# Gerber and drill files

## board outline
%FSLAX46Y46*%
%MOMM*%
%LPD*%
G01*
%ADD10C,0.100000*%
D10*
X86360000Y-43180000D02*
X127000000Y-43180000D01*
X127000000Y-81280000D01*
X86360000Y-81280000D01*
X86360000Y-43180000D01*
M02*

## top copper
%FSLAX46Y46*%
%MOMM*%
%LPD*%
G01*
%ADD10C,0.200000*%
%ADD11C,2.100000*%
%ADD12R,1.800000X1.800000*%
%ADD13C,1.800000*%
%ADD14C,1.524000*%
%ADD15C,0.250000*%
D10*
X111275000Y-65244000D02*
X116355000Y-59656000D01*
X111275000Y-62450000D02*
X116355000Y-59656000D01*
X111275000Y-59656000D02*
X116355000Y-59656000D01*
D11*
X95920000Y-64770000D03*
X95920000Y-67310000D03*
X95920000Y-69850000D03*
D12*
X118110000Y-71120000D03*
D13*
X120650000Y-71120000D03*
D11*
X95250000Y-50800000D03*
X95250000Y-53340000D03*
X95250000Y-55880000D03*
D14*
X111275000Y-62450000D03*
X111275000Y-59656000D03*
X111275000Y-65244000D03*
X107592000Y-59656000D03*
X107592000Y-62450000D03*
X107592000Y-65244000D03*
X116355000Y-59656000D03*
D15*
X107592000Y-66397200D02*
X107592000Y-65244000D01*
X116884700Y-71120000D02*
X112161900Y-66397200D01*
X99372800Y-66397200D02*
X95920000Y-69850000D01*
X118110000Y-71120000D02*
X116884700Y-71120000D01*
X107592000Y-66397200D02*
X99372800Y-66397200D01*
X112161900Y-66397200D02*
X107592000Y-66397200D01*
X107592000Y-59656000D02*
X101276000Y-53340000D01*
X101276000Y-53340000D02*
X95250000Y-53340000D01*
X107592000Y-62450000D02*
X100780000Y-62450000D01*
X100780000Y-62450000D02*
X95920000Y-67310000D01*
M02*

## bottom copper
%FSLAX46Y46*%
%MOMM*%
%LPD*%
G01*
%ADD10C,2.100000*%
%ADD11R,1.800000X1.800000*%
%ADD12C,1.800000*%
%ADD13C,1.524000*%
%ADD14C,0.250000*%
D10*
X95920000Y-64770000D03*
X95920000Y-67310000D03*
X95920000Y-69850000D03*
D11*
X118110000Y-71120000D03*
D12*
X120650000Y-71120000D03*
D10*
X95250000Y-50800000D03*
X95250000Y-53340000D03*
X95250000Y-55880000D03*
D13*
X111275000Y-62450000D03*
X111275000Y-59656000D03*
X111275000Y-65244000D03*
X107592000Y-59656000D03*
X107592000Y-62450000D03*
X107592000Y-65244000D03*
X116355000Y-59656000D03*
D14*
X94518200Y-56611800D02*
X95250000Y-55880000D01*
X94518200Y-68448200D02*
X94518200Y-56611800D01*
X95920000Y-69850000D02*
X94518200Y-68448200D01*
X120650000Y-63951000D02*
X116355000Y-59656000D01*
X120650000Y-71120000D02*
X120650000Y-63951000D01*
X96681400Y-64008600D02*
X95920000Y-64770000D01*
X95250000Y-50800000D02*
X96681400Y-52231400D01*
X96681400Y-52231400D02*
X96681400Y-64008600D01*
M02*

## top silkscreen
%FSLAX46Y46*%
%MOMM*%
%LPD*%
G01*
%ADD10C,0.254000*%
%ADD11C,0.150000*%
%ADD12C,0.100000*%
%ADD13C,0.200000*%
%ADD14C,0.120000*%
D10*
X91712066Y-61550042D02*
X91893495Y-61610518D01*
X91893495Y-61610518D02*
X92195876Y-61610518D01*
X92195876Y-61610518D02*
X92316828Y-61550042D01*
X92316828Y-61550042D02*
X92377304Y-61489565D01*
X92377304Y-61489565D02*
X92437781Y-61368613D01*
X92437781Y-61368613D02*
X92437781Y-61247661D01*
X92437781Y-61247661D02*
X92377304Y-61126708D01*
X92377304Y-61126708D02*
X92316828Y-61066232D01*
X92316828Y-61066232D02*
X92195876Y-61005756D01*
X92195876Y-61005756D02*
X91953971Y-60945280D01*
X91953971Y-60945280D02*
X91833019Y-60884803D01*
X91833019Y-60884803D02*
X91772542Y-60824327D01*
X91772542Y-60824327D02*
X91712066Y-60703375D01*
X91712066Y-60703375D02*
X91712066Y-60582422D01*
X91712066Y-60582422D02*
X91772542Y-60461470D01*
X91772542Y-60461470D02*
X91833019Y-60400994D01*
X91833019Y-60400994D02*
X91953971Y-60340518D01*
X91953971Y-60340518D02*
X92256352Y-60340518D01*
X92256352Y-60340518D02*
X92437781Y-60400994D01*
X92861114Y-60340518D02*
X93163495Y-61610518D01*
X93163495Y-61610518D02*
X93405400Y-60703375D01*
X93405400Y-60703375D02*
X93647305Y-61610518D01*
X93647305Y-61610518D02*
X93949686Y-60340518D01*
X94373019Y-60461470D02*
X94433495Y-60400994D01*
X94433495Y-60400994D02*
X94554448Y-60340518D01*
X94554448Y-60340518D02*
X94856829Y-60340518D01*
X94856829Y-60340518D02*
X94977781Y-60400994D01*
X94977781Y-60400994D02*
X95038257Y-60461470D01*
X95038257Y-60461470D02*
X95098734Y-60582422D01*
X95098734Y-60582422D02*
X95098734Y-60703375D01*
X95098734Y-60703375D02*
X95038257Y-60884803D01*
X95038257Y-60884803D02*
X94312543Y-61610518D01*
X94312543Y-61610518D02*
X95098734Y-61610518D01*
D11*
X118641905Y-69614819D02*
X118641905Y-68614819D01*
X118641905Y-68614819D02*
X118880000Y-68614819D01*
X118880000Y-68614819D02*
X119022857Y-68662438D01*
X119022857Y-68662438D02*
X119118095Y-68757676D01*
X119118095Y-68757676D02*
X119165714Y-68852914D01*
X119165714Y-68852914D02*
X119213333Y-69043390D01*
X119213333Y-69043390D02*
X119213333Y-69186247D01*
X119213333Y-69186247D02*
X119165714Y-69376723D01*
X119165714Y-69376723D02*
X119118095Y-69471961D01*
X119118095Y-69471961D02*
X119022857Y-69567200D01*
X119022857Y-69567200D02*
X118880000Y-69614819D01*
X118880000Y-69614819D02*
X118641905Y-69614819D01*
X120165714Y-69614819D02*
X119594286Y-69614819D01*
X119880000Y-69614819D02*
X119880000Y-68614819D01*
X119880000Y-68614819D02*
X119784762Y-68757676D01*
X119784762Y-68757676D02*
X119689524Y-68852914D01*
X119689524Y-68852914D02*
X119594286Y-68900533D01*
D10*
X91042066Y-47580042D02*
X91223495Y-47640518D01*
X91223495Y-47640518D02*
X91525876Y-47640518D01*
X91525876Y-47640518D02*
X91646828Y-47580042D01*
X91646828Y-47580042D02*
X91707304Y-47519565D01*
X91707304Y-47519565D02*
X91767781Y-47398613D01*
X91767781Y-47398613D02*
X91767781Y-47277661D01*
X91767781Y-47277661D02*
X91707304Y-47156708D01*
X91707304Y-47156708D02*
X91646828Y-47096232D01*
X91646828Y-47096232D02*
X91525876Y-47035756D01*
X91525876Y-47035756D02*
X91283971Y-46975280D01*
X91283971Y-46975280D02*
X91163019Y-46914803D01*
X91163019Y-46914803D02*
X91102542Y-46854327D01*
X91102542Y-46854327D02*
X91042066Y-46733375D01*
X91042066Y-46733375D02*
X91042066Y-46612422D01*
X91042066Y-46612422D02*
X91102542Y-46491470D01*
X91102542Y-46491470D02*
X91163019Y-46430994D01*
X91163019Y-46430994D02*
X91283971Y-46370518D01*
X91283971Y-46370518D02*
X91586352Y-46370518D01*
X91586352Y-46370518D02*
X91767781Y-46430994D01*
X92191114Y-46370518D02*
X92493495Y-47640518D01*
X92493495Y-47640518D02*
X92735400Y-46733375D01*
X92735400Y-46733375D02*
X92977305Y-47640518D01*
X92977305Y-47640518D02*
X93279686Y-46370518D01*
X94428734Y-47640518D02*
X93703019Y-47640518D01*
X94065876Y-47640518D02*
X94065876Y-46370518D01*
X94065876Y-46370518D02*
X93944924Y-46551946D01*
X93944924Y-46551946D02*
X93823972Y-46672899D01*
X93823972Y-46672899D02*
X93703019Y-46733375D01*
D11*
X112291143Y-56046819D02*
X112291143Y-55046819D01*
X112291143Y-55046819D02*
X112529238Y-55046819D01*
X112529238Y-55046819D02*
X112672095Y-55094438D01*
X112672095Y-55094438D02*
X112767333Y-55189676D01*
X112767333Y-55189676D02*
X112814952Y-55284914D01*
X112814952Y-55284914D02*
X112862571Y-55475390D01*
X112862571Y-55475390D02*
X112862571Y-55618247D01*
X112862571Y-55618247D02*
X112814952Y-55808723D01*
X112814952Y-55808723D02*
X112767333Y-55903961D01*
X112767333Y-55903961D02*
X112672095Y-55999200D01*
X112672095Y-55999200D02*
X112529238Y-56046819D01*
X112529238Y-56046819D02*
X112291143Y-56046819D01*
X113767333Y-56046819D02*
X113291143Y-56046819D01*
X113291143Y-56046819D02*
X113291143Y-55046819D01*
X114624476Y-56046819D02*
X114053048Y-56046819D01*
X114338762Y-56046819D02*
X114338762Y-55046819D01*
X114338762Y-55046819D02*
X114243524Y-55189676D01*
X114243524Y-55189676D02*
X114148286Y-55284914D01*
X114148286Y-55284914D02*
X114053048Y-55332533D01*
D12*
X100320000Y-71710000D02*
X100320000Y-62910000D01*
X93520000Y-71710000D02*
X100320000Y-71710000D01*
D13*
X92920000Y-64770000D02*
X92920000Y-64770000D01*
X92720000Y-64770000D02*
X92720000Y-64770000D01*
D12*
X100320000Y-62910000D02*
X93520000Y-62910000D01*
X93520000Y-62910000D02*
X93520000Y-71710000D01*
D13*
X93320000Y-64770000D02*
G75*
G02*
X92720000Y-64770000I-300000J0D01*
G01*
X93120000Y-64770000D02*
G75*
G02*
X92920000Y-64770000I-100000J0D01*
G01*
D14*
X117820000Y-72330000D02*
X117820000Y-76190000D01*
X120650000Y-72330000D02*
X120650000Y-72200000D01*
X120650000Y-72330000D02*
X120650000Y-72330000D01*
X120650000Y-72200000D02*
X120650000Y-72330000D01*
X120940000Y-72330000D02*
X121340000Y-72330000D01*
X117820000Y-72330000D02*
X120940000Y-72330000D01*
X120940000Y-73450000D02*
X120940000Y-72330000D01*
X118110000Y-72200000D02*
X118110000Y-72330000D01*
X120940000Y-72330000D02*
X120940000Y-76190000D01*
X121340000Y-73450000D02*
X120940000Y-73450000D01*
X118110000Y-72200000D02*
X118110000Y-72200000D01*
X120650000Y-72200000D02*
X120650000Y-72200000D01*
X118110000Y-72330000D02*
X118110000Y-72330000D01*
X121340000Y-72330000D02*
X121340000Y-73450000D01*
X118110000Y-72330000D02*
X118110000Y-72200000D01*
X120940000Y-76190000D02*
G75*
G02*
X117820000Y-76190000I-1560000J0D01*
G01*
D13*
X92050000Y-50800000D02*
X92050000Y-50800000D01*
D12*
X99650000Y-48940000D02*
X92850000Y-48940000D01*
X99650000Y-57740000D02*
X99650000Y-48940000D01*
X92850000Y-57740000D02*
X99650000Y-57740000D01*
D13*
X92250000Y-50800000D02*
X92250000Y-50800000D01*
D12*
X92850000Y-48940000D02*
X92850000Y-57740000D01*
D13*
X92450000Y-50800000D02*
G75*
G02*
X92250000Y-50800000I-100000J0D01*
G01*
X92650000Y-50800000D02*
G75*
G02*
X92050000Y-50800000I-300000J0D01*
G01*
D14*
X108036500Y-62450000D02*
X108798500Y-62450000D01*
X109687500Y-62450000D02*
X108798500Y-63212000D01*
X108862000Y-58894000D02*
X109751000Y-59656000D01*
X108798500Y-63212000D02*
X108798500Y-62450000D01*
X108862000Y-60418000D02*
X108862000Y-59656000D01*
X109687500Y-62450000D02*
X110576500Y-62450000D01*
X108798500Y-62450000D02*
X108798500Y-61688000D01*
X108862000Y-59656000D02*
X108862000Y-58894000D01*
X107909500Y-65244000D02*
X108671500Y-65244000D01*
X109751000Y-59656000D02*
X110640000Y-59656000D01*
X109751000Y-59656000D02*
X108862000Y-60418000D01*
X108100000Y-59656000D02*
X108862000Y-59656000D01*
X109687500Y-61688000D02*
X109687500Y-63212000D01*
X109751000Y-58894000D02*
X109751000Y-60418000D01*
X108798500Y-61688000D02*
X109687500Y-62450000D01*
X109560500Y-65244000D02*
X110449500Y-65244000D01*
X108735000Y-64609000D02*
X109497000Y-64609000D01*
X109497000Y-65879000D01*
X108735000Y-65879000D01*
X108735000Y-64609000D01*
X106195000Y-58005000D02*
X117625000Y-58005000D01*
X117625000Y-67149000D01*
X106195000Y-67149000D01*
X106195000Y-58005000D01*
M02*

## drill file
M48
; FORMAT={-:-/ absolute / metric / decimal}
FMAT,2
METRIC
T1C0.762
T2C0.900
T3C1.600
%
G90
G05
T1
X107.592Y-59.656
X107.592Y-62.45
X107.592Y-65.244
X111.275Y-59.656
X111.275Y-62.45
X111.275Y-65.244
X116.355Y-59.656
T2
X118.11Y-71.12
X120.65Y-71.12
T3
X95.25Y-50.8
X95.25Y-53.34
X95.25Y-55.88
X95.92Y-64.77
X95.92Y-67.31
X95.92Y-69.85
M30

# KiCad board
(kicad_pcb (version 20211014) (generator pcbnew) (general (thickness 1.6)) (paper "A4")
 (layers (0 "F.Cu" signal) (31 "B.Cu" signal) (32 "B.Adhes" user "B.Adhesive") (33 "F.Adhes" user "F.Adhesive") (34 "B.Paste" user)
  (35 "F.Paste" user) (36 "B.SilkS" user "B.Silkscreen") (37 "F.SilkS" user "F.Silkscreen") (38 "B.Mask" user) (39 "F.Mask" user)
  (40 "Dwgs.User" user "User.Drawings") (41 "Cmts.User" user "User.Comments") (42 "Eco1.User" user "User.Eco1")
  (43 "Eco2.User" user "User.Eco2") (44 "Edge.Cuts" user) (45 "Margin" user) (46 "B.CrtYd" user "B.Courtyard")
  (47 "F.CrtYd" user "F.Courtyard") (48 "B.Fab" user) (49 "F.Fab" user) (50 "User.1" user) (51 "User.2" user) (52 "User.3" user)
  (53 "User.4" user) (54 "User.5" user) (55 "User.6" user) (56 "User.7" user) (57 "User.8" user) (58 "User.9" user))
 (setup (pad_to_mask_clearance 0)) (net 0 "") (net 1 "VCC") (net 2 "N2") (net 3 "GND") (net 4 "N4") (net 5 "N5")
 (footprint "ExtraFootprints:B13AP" (layer "F.Cu") (at 95.92 64.77)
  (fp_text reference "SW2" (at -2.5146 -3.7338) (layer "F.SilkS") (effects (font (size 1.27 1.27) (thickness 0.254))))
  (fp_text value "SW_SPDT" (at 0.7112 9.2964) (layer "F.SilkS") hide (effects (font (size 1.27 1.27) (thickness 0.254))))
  (fp_line (start 4.4 6.94) (end 4.4 -1.86) (layer "F.SilkS") (width 0.1))
  (fp_line (start -2.4 6.94) (end 4.4 6.94) (layer "F.SilkS") (width 0.1))
  (fp_line (start -3 0) (end -3 0) (layer "F.SilkS") (width 0.2))
  (fp_line (start -3.2 0) (end -3.2 0) (layer "F.SilkS") (width 0.2))
  (fp_line (start 4.4 -1.86) (end -2.4 -1.86) (layer "F.SilkS") (width 0.1))
  (fp_line (start -2.4 -1.86) (end -2.4 6.94) (layer "F.SilkS") (width 0.1))
  (fp_arc (start -2.6 0) (mid -2.9 0.3) (end -3.2 0) (layer "F.SilkS") (width 0.2))
  (fp_arc (start -2.8 0) (mid -2.9 0.1) (end -3 0) (layer "F.SilkS") (width 0.2))
  (pad "1" thru_hole circle (at 0 0 90) (size 2.1 2.1) (drill 1.6) (layers *.Cu *.Mask) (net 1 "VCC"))
  (pad "2" thru_hole circle (at 0 2.54 90) (size 2.1 2.1) (drill 1.6) (layers *.Cu *.Mask) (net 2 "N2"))
  (pad "3" thru_hole circle (at 0 5.08 90) (size 2.1 2.1) (drill 1.6) (layers *.Cu *.Mask) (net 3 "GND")))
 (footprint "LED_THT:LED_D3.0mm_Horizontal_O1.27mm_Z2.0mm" (layer "F.Cu") (at 118.11 71.12)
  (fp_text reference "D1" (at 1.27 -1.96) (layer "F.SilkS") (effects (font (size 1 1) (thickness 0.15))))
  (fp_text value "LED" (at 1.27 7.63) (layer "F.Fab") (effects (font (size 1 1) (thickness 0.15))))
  (fp_line (start -0.29 1.21) (end -0.29 5.07) (layer "F.SilkS") (width 0.12))
  (fp_line (start 2.54 1.21) (end 2.54 1.08) (layer "F.SilkS") (width 0.12))
  (fp_line (start 2.54 1.21) (end 2.54 1.21) (layer "F.SilkS") (width 0.12))
  (fp_line (start 2.54 1.08) (end 2.54 1.21) (layer "F.SilkS") (width 0.12))
  (fp_line (start 2.83 1.21) (end 3.23 1.21) (layer "F.SilkS") (width 0.12))
  (fp_line (start -0.29 1.21) (end 2.83 1.21) (layer "F.SilkS") (width 0.12))
  (fp_line (start 2.83 2.33) (end 2.83 1.21) (layer "F.SilkS") (width 0.12))
  (fp_line (start 0 1.08) (end 0 1.21) (layer "F.SilkS") (width 0.12))
  (fp_line (start 2.83 1.21) (end 2.83 5.07) (layer "F.SilkS") (width 0.12))
  (fp_line (start 3.23 2.33) (end 2.83 2.33) (layer "F.SilkS") (width 0.12))
  (fp_line (start 0 1.08) (end 0 1.08) (layer "F.SilkS") (width 0.12))
  (fp_line (start 2.54 1.08) (end 2.54 1.08) (layer "F.SilkS") (width 0.12))
  (fp_line (start 0 1.21) (end 0 1.21) (layer "F.SilkS") (width 0.12))
  (fp_line (start 3.23 1.21) (end 3.23 2.33) (layer "F.SilkS") (width 0.12))
  (fp_line (start 0 1.21) (end 0 1.08) (layer "F.SilkS") (width 0.12))
  (fp_arc (start 2.83 5.07) (mid 1.27 6.63) (end -0.29 5.07) (layer "F.SilkS") (width 0.12))
  (pad "1" thru_hole rect (at 0 0) (size 1.8 1.8) (drill 0.9) (layers *.Cu *.Mask) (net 3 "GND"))
  (pad "2" thru_hole circle (at 2.54 0) (size 1.8 1.8) (drill 0.9) (layers *.Cu *.Mask) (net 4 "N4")))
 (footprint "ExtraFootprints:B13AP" (layer "F.Cu") (at 95.25 50.8)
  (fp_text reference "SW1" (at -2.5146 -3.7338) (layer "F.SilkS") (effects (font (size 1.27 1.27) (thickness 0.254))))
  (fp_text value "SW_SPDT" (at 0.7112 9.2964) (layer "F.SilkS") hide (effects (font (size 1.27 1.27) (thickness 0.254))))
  (fp_line (start -3.2 0) (end -3.2 0) (layer "F.SilkS") (width 0.2))
  (fp_line (start 4.4 -1.86) (end -2.4 -1.86) (layer "F.SilkS") (width 0.1))
  (fp_line (start 4.4 6.94) (end 4.4 -1.86) (layer "F.SilkS") (width 0.1))
  (fp_line (start -2.4 6.94) (end 4.4 6.94) (layer "F.SilkS") (width 0.1))
  (fp_line (start -3 0) (end -3 0) (layer "F.SilkS") (width 0.2))
  (fp_line (start -2.4 -1.86) (end -2.4 6.94) (layer "F.SilkS") (width 0.1))
  (fp_arc (start -2.8 0) (mid -2.9 0.1) (end -3 0) (layer "F.SilkS") (width 0.2))
  (fp_arc (start -2.6 0) (mid -2.9 0.3) (end -3.2 0) (layer "F.SilkS") (width 0.2))
  (pad "1" thru_hole circle (at 0 0 90) (size 2.1 2.1) (drill 1.6) (layers *.Cu *.Mask) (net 1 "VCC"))
  (pad "2" thru_hole circle (at 0 2.54 90) (size 2.1 2.1) (drill 1.6) (layers *.Cu *.Mask) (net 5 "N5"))
  (pad "3" thru_hole circle (at 0 5.08 90) (size 2.1 2.1) (drill 1.6) (layers *.Cu *.Mask) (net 3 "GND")))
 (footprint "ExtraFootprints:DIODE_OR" (layer "F.Cu") (at 107.592 59.656)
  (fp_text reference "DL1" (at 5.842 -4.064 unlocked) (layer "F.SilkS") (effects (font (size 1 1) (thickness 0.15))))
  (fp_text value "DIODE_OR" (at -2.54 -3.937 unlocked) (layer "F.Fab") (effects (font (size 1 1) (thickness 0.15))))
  (fp_line (start 3.683 5.588) (end 8.763 0) (layer "F.Cu") (width 0.2))
  (fp_line (start 3.683 2.794) (end 8.763 0) (layer "F.Cu") (width 0.2))
  (fp_line (start 3.683 0) (end 8.763 0) (layer "F.Cu") (width 0.2))
  (fp_line (start 0.4445 2.794) (end 1.2065 2.794) (layer "F.SilkS") (width 0.12))
  (fp_line (start 2.0955 2.794) (end 1.2065 3.556) (layer "F.SilkS") (width 0.12))
  (fp_line (start 1.27 -0.762) (end 2.159 0) (layer "F.SilkS") (width 0.12))
  (fp_line (start 1.2065 3.556) (end 1.2065 2.794) (layer "F.SilkS") (width 0.12))
  (fp_line (start 1.27 0.762) (end 1.27 0) (layer "F.SilkS") (width 0.12))
  (fp_line (start 2.0955 2.794) (end 2.9845 2.794) (layer "F.SilkS") (width 0.12))
  (fp_line (start 1.2065 2.794) (end 1.2065 2.032) (layer "F.SilkS") (width 0.12))
  (fp_line (start 1.27 0) (end 1.27 -0.762) (layer "F.SilkS") (width 0.12))
  (fp_line (start 0.3175 5.588) (end 1.0795 5.588) (layer "F.SilkS") (width 0.12))
  (fp_line (start 2.159 0) (end 3.048 0) (layer "F.SilkS") (width 0.12))
  (fp_line (start 2.159 0) (end 1.27 0.762) (layer "F.SilkS") (width 0.12))
  (fp_line (start 0.508 0) (end 1.27 0) (layer "F.SilkS") (width 0.12))
  (fp_line (start 2.0955 2.032) (end 2.0955 3.556) (layer "F.SilkS") (width 0.12))
  (fp_line (start 2.159 -0.762) (end 2.159 0.762) (layer "F.SilkS") (width 0.12))
  (fp_line (start 1.2065 2.032) (end 2.0955 2.794) (layer "F.SilkS") (width 0.12))
  (fp_line (start 1.9685 5.588) (end 2.8575 5.588) (layer "F.SilkS") (width 0.12))
  (fp_rect (start 1.143 4.953) (end 1.905 6.223) (layer "F.SilkS") (width 0.12) (fill none))
  (fp_rect (start -1.397 -1.651) (end 10.033 7.493) (layer "F.SilkS") (width 0.12) (fill none))
  (pad "" thru_hole circle (at 3.683 2.794) (size 1.524 1.524) (drill 0.762) (layers *.Cu *.Mask))
  (pad "" thru_hole circle (at 3.683 0) (size 1.524 1.524) (drill 0.762) (layers *.Cu *.Mask))
  (pad "" thru_hole circle (at 3.683 5.588) (size 1.524 1.524) (drill 0.762) (layers *.Cu *.Mask))
  (pad "1" thru_hole circle (at 0 0) (size 1.524 1.524) (drill 0.762) (layers *.Cu *.Mask) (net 5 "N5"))
  (pad "2" thru_hole circle (at 0 2.794) (size 1.524 1.524) (drill 0.762) (layers *.Cu *.Mask) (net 2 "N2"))
  (pad "3" thru_hole circle (at 0 5.588) (size 1.524 1.524) (drill 0.762) (layers *.Cu *.Mask) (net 3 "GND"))
  (pad "4" thru_hole circle (at 8.763 0) (size 1.524 1.524) (drill 0.762) (layers *.Cu *.Mask) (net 4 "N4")))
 (gr_rect (start 86.36 43.18) (end 127 81.28) (layer "Edge.Cuts") (width 0.1) (fill none))
 (segment (start 107.592 66.3972) (end 107.592 65.244) (width 0.25) (layer "F.Cu") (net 3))
 (segment (start 116.8847 71.12) (end 112.1619 66.3972) (width 0.25) (layer "F.Cu") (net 3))
 (segment (start 99.3728 66.3972) (end 95.92 69.85) (width 0.25) (layer "F.Cu") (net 3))
 (segment (start 118.11 71.12) (end 116.8847 71.12) (width 0.25) (layer "F.Cu") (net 3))
 (segment (start 107.592 66.3972) (end 99.3728 66.3972) (width 0.25) (layer "F.Cu") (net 3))
 (segment (start 112.1619 66.3972) (end 107.592 66.3972) (width 0.25) (layer "F.Cu") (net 3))
 (segment (start 94.5182 56.6118) (end 95.25 55.88) (width 0.25) (layer "B.Cu") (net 3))
 (segment (start 94.5182 68.4482) (end 94.5182 56.6118) (width 0.25) (layer "B.Cu") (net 3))
 (segment (start 95.92 69.85) (end 94.5182 68.4482) (width 0.25) (layer "B.Cu") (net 3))
 (segment (start 120.65 63.951) (end 116.355 59.656) (width 0.25) (layer "B.Cu") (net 4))
 (segment (start 120.65 71.12) (end 120.65 63.951) (width 0.25) (layer "B.Cu") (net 4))
 (segment (start 107.592 59.656) (end 101.276 53.34) (width 0.25) (layer "F.Cu") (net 5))
 (segment (start 101.276 53.34) (end 95.25 53.34) (width 0.25) (layer "F.Cu") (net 5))
 (segment (start 107.592 62.45) (end 100.78 62.45) (width 0.25) (layer "F.Cu") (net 2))
 (segment (start 100.78 62.45) (end 95.92 67.31) (width 0.25) (layer "F.Cu") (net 2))
 (segment (start 96.6814 64.0086) (end 95.92 64.77) (width 0.25) (layer "B.Cu") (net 1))
 (segment (start 95.25 50.8) (end 96.6814 52.2314) (width 0.25) (layer "B.Cu") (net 1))
 (segment (start 96.6814 52.2314) (end 96.6814 64.0086) (width 0.25) (layer "B.Cu") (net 1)))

